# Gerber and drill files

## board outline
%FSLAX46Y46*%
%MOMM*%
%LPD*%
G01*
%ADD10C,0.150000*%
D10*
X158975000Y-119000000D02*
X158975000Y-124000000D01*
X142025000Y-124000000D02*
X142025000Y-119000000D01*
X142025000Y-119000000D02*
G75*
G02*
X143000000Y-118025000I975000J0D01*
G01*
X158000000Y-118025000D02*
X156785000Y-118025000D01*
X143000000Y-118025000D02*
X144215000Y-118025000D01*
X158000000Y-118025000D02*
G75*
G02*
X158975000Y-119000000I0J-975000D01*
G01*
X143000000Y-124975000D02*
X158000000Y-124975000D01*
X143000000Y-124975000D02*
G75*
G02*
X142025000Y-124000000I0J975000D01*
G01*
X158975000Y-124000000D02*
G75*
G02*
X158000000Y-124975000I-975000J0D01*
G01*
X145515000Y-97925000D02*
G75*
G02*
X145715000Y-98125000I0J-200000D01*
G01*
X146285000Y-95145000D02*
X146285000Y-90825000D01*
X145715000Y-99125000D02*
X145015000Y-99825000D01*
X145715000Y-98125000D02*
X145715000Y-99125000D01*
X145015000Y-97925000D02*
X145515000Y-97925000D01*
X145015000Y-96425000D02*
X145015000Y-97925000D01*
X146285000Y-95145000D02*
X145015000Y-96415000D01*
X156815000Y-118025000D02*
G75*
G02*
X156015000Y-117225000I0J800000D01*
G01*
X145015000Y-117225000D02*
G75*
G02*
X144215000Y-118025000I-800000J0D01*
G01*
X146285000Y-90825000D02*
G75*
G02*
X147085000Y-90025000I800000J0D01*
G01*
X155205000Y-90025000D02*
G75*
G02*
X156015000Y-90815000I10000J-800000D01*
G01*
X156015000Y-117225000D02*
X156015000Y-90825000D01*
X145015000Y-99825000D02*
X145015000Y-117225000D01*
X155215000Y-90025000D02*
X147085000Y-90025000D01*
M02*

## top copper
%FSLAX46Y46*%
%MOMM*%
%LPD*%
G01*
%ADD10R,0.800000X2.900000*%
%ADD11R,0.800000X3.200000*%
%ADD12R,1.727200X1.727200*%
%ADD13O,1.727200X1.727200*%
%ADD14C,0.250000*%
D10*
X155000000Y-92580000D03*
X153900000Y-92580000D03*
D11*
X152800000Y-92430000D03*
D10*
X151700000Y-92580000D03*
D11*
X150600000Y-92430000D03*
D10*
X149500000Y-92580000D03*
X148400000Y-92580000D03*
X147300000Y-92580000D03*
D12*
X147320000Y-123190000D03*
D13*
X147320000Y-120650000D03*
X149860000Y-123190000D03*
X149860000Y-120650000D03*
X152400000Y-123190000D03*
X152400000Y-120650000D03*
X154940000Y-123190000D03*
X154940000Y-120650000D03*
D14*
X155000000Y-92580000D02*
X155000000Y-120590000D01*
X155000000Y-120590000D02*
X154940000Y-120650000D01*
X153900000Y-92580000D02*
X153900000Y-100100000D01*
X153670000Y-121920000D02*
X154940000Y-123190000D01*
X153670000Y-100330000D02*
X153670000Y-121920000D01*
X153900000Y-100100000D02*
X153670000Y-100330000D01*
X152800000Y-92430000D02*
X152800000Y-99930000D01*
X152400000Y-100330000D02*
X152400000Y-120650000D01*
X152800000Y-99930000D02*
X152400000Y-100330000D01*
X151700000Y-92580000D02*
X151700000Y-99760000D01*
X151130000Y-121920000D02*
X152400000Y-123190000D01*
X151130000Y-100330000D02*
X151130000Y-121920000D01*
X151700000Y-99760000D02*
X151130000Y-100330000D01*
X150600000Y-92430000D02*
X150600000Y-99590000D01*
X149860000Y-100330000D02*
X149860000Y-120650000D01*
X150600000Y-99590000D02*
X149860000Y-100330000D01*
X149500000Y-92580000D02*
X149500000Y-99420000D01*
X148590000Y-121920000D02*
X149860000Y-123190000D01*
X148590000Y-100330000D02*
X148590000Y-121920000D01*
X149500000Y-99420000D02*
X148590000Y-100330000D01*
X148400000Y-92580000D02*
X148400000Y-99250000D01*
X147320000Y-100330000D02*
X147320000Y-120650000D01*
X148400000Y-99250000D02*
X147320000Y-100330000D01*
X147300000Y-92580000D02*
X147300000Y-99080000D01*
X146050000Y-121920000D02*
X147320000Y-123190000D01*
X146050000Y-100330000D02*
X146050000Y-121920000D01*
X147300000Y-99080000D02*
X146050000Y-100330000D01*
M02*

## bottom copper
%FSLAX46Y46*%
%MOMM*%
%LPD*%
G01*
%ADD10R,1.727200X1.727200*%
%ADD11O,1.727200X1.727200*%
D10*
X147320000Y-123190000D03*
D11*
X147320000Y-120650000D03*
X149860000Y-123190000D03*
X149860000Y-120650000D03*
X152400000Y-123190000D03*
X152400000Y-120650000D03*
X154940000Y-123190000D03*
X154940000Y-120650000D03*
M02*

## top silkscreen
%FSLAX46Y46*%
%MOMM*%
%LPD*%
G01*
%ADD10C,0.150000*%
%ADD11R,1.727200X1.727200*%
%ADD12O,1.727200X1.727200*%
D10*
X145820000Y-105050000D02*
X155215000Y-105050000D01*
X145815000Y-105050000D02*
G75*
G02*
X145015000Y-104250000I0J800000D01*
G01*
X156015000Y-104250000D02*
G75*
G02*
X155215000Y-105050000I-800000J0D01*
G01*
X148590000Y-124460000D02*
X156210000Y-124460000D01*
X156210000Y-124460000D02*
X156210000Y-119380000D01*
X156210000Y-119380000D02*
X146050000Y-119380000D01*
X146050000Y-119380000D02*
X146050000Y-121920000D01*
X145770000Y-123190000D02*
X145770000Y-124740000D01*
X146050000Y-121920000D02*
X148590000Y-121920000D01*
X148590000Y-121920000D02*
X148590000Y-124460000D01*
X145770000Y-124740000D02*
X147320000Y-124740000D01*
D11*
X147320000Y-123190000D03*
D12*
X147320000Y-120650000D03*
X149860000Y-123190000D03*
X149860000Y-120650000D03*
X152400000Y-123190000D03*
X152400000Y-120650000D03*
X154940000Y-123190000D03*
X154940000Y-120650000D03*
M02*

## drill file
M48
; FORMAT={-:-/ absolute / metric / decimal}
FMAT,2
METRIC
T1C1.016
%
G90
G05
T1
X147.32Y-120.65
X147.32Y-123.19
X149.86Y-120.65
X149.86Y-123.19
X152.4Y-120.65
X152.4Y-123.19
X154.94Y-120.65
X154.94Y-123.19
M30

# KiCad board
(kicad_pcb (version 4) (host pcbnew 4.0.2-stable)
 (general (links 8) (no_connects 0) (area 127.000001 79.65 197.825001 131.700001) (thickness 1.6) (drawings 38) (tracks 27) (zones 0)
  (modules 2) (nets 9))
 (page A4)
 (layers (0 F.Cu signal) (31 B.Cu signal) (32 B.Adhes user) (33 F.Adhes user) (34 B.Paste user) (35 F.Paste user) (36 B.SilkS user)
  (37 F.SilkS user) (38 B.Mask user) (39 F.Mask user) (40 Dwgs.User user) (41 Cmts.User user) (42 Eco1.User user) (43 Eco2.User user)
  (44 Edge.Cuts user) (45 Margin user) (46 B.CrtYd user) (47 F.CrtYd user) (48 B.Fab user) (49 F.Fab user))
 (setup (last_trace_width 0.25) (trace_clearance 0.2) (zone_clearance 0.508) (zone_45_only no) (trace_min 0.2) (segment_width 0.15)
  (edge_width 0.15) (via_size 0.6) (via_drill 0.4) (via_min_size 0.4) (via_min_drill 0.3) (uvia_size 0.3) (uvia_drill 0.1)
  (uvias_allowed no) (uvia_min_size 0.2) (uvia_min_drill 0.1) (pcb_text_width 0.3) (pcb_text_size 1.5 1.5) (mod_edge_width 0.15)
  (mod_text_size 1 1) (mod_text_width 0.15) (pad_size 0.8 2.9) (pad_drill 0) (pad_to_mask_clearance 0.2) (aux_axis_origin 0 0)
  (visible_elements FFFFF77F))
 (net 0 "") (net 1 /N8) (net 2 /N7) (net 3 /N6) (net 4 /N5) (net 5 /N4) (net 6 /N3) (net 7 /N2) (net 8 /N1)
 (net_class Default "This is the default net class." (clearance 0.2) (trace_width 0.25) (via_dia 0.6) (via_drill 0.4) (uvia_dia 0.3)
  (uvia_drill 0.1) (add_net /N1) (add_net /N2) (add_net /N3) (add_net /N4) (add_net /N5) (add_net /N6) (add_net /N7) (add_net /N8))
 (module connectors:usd (layer F.Cu) (at 147.3 92.58)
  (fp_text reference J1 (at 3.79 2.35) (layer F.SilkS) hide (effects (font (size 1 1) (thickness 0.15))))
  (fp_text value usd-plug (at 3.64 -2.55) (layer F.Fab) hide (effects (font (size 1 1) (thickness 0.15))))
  (pad 8 smd rect (at 7.7 0) (size 0.8 2.9) (layers F.Cu F.Paste F.Mask) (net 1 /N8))
  (pad 7 smd rect (at 6.6 0) (size 0.8 2.9) (layers F.Cu F.Paste F.Mask) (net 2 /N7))
  (pad 6 smd rect (at 5.5 -0.15) (size 0.8 3.2) (layers F.Cu F.Paste F.Mask) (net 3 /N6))
  (pad 5 smd rect (at 4.4 0) (size 0.8 2.9) (layers F.Cu F.Paste F.Mask) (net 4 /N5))
  (pad 4 smd rect (at 3.3 -0.15) (size 0.8 3.2) (layers F.Cu F.Paste F.Mask) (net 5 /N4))
  (pad 3 smd rect (at 2.2 0) (size 0.8 2.9) (layers F.Cu F.Paste F.Mask) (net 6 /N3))
  (pad 2 smd rect (at 1.1 0) (size 0.8 2.9) (layers F.Cu F.Paste F.Mask) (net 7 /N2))
  (pad 1 smd rect (at 0 0) (size 0.8 2.9) (layers F.Cu F.Paste F.Mask) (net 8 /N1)))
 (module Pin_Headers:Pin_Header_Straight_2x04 (layer F.Cu) (at 147.32 123.19 90)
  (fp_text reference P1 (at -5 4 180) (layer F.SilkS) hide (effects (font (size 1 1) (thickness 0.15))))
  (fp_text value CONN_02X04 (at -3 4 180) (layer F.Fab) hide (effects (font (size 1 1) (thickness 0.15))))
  (fp_line (start -1.27 1.27) (end -1.27 8.89) (layer F.SilkS) (width 0.15))
  (fp_line (start -1.27 8.89) (end 3.81 8.89) (layer F.SilkS) (width 0.15))
  (fp_line (start 3.81 8.89) (end 3.81 -1.27) (layer F.SilkS) (width 0.15))
  (fp_line (start 3.81 -1.27) (end 1.27 -1.27) (layer F.SilkS) (width 0.15))
  (fp_line (start 0 -1.55) (end -1.55 -1.55) (layer F.SilkS) (width 0.15))
  (fp_line (start 1.27 -1.27) (end 1.27 1.27) (layer F.SilkS) (width 0.15))
  (fp_line (start 1.27 1.27) (end -1.27 1.27) (layer F.SilkS) (width 0.15))
  (fp_line (start -1.55 -1.55) (end -1.55 0) (layer F.SilkS) (width 0.15))
  (pad 1 thru_hole rect (at 0 0 90) (size 1.7272 1.7272) (drill 1.016) (layers *.Cu *.Mask F.SilkS) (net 8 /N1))
  (pad 2 thru_hole oval (at 2.54 0 90) (size 1.7272 1.7272) (drill 1.016) (layers *.Cu *.Mask F.SilkS) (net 7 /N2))
  (pad 3 thru_hole oval (at 0 2.54 90) (size 1.7272 1.7272) (drill 1.016) (layers *.Cu *.Mask F.SilkS) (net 6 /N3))
  (pad 4 thru_hole oval (at 2.54 2.54 90) (size 1.7272 1.7272) (drill 1.016) (layers *.Cu *.Mask F.SilkS) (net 5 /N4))
  (pad 5 thru_hole oval (at 0 5.08 90) (size 1.7272 1.7272) (drill 1.016) (layers *.Cu *.Mask F.SilkS) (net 4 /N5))
  (pad 6 thru_hole oval (at 2.54 5.08 90) (size 1.7272 1.7272) (drill 1.016) (layers *.Cu *.Mask F.SilkS) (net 3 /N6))
  (pad 7 thru_hole oval (at 0 7.62 90) (size 1.7272 1.7272) (drill 1.016) (layers *.Cu *.Mask F.SilkS) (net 2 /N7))
  (pad 8 thru_hole oval (at 2.54 7.62 90) (size 1.7272 1.7272) (drill 1.016) (layers *.Cu *.Mask F.SilkS) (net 1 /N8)))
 (gr_line (start 158.975 119) (end 158.975 124) (angle 90) (layer Edge.Cuts) (width 0.15))
 (gr_line (start 142.025 124) (end 142.025 119) (angle 90) (layer Edge.Cuts) (width 0.15))
 (gr_arc (start 143 119) (end 143 118.025) (angle -90) (layer Edge.Cuts) (width 0.15))
 (gr_line (start 158 118.025) (end 156.785 118.025) (angle 90) (layer Edge.Cuts) (width 0.15))
 (gr_line (start 143 118.025) (end 144.215 118.025) (angle 90) (layer Edge.Cuts) (width 0.15))
 (gr_arc (start 158 119) (end 158 118.025) (angle 90) (layer Edge.Cuts) (width 0.15))
 (gr_line (start 143 124.975) (end 158 124.975) (angle 90) (layer Edge.Cuts) (width 0.15))
 (gr_arc (start 143 124) (end 143 124.975) (angle 90) (layer Edge.Cuts) (width 0.15))
 (gr_arc (start 158 124) (end 158.975 124) (angle 90) (layer Edge.Cuts) (width 0.15))
 (gr_line (start 145.82 105.05) (end 155.215 105.05) (angle 90) (layer F.SilkS) (width 0.15))
 (gr_arc (start 145.815 104.25) (end 145.815 105.05) (angle 90) (layer F.SilkS) (width 0.15))
 (gr_arc (start 155.215 104.25) (end 156.015 104.25) (angle 90) (layer F.SilkS) (width 0.15))
 (gr_arc (start 145.515 98.125) (end 145.715 98.125) (angle -90) (layer Edge.Cuts) (width 0.15))
 (gr_line (start 146.285 95.145) (end 146.285 90.825) (angle 90) (layer Edge.Cuts) (width 0.15))
 (gr_line (start 145.715 99.125) (end 145.015 99.825) (angle 90) (layer Edge.Cuts) (width 0.15))
 (gr_line (start 145.715 98.125) (end 145.715 99.125) (angle 90) (layer Edge.Cuts) (width 0.15))
 (gr_line (start 145.015 97.925) (end 145.515 97.925) (angle 90) (layer Edge.Cuts) (width 0.15))
 (gr_line (start 145.015 96.425) (end 145.015 97.925) (angle 90) (layer Edge.Cuts) (width 0.15))
 (gr_line (start 146.285 95.145) (end 145.015 96.415) (angle 90) (layer Edge.Cuts) (width 0.15))
 (gr_arc (start 156.815 117.225) (end 156.815 118.025) (angle 90) (layer Edge.Cuts) (width 0.15))
 (gr_arc (start 144.215 117.225) (end 145.015 117.225) (angle 90) (layer Edge.Cuts) (width 0.15))
 (gr_arc (start 147.085 90.825) (end 147.085 90.025) (angle -90) (layer Edge.Cuts) (width 0.15))
 (gr_arc (start 155.215 90.825) (end 156.015 90.815) (angle -90) (layer Edge.Cuts) (width 0.15))
 (gr_line (start 156.015 117.225) (end 156.015 90.825) (angle 90) (layer Edge.Cuts) (width 0.15))
 (gr_line (start 145.015 99.825) (end 145.015 117.225) (angle 90) (layer Edge.Cuts) (width 0.15))
 (gr_line (start 155.215 90.025) (end 147.085 90.025) (angle 90) (layer Edge.Cuts) (width 0.15))
 (segment (start 155 92.58) (end 155 120.59) (width 0.25) (layer F.Cu) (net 1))
 (segment (start 155 120.59) (end 154.94 120.65) (width 0.25) (layer F.Cu) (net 1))
 (segment (start 153.9 92.58) (end 153.9 100.1) (width 0.25) (layer F.Cu) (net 2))
 (segment (start 153.67 121.92) (end 154.94 123.19) (width 0.25) (layer F.Cu) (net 2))
 (segment (start 153.67 100.33) (end 153.67 121.92) (width 0.25) (layer F.Cu) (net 2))
 (segment (start 153.9 100.1) (end 153.67 100.33) (width 0.25) (layer F.Cu) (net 2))
 (segment (start 152.8 92.43) (end 152.8 99.93) (width 0.25) (layer F.Cu) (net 3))
 (segment (start 152.4 100.33) (end 152.4 120.65) (width 0.25) (layer F.Cu) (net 3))
 (segment (start 152.8 99.93) (end 152.4 100.33) (width 0.25) (layer F.Cu) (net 3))
 (segment (start 151.7 92.58) (end 151.7 99.76) (width 0.25) (layer F.Cu) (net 4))
 (segment (start 151.13 121.92) (end 152.4 123.19) (width 0.25) (layer F.Cu) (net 4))
 (segment (start 151.13 100.33) (end 151.13 121.92) (width 0.25) (layer F.Cu) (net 4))
 (segment (start 151.7 99.76) (end 151.13 100.33) (width 0.25) (layer F.Cu) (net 4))
 (segment (start 150.6 92.43) (end 150.6 99.59) (width 0.25) (layer F.Cu) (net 5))
 (segment (start 149.86 100.33) (end 149.86 120.65) (width 0.25) (layer F.Cu) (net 5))
 (segment (start 150.6 99.59) (end 149.86 100.33) (width 0.25) (layer F.Cu) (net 5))
 (segment (start 149.5 92.58) (end 149.5 99.42) (width 0.25) (layer F.Cu) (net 6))
 (segment (start 148.59 121.92) (end 149.86 123.19) (width 0.25) (layer F.Cu) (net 6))
 (segment (start 148.59 100.33) (end 148.59 121.92) (width 0.25) (layer F.Cu) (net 6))
 (segment (start 149.5 99.42) (end 148.59 100.33) (width 0.25) (layer F.Cu) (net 6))
 (segment (start 148.4 92.58) (end 148.4 99.25) (width 0.25) (layer F.Cu) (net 7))
 (segment (start 147.32 100.33) (end 147.32 120.65) (width 0.25) (layer F.Cu) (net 7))
 (segment (start 148.4 99.25) (end 147.32 100.33) (width 0.25) (layer F.Cu) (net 7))
 (segment (start 147.3 92.58) (end 147.3 99.08) (width 0.25) (layer F.Cu) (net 8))
 (segment (start 146.05 121.92) (end 147.32 123.19) (width 0.25) (layer F.Cu) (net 8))
 (segment (start 146.05 100.33) (end 146.05 121.92) (width 0.25) (layer F.Cu) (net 8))
 (segment (start 147.3 99.08) (end 146.05 100.33) (width 0.25) (layer F.Cu) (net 8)))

